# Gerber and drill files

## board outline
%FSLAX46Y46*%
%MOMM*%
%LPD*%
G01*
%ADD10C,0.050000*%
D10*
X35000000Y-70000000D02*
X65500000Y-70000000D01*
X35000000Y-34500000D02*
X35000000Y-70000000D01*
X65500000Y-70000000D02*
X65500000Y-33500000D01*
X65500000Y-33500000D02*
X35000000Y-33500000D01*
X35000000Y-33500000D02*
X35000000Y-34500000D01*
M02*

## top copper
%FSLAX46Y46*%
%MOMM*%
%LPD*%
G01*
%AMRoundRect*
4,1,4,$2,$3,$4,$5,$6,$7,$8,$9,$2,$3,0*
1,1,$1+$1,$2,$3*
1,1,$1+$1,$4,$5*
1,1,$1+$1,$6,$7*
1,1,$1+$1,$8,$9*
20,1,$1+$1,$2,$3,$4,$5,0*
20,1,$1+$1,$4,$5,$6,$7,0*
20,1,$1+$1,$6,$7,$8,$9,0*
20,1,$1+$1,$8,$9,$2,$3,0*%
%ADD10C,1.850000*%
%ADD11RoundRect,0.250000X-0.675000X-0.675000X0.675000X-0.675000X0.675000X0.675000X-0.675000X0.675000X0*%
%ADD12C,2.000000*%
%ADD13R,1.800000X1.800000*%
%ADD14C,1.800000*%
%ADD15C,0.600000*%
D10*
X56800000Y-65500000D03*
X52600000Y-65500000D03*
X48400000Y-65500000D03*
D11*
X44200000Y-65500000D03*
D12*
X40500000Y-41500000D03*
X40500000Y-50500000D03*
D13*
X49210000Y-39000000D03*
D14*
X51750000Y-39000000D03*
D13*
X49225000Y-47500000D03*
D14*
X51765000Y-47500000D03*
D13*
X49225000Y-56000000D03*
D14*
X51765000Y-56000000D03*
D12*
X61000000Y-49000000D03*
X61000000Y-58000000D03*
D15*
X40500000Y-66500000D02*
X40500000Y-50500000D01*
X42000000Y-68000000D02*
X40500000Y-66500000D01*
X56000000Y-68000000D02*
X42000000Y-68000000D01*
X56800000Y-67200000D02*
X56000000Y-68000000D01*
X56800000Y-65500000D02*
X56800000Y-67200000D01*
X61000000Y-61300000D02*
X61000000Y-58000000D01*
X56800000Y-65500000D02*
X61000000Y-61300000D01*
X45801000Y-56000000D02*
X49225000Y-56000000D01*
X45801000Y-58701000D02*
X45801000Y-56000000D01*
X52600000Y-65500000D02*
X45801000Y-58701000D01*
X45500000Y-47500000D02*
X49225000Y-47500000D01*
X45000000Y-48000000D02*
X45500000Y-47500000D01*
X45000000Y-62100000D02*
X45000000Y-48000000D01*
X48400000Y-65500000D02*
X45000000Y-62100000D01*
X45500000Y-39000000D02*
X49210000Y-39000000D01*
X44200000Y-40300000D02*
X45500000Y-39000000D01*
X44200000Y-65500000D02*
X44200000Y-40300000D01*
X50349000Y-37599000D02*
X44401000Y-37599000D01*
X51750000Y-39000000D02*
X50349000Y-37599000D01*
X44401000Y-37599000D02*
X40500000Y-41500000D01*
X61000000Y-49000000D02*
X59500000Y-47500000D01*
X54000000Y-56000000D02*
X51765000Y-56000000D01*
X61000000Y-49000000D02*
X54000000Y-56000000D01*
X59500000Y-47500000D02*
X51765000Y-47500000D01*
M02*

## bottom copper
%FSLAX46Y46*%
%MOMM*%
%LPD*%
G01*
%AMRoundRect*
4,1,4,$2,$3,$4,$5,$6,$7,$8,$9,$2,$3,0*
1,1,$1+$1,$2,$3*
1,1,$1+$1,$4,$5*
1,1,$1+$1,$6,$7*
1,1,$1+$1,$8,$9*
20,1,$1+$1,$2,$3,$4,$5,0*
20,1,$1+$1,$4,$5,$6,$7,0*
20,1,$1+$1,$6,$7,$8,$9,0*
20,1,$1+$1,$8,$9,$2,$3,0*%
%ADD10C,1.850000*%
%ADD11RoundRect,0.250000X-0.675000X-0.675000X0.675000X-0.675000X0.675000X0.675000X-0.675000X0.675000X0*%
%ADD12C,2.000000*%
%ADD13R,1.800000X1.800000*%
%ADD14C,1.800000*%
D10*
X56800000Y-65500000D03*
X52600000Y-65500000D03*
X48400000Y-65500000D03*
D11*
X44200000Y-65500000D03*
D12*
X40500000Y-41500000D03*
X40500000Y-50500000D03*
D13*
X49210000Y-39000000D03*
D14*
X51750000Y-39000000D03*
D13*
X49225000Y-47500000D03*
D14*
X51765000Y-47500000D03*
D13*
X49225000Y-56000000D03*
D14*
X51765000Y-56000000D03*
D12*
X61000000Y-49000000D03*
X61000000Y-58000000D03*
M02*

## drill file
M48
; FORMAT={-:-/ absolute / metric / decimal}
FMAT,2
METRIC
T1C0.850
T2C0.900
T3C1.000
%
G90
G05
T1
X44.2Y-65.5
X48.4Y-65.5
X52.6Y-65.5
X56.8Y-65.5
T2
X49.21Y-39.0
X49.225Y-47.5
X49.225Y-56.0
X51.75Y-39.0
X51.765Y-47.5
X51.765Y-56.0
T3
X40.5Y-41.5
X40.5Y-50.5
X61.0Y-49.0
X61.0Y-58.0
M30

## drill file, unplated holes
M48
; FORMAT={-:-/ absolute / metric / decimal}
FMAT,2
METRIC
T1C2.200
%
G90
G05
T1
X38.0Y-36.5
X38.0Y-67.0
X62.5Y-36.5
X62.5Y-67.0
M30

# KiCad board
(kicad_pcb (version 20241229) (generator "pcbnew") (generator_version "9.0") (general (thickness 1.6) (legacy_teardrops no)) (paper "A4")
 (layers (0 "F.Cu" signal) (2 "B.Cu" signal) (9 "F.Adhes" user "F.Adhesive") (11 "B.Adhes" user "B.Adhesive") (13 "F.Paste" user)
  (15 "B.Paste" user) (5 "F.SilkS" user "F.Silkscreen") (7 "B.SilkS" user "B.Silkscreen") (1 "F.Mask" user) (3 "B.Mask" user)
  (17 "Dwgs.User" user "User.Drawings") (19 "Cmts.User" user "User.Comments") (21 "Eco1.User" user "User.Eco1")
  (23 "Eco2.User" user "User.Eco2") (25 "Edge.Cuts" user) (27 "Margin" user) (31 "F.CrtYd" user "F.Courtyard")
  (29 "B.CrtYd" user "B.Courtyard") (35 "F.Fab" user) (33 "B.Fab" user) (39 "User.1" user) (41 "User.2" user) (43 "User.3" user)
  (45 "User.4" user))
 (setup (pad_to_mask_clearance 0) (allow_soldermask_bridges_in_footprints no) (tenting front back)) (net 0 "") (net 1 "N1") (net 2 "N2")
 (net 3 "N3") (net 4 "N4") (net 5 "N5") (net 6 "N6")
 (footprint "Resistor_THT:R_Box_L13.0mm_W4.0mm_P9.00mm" (layer "F.Cu") (at 40.5 41.5 -90)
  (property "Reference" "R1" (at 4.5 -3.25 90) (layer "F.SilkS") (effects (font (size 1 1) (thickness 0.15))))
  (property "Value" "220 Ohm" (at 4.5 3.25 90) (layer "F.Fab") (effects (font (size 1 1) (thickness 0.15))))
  (pad "1" thru_hole circle (at 0 0 270) (size 2 2) (drill 1) (layers "*.Cu" "*.Mask") (remove_unused_layers no) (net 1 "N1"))
  (pad "2" thru_hole circle (at 9 0 270) (size 2 2) (drill 1) (layers "*.Cu" "*.Mask") (remove_unused_layers no) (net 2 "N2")))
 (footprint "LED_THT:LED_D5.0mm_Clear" (layer "F.Cu") (at 49.21 39)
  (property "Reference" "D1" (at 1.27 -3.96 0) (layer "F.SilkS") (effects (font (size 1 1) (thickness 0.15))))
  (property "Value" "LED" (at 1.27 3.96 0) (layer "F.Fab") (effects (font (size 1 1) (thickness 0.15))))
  (pad "1" thru_hole rect (at 0 0) (size 1.8 1.8) (drill 0.9) (layers "*.Cu" "*.Mask") (remove_unused_layers no) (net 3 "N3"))
  (pad "2" thru_hole circle (at 2.54 0) (size 1.8 1.8) (drill 0.9) (layers "*.Cu" "*.Mask") (remove_unused_layers no) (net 1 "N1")))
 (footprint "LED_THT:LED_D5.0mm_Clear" (layer "F.Cu") (at 49.225 47.5)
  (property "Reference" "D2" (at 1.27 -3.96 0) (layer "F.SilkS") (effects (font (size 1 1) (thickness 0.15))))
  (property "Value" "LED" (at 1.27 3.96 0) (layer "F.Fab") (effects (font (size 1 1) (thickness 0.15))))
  (pad "1" thru_hole rect (at 0 0) (size 1.8 1.8) (drill 0.9) (layers "*.Cu" "*.Mask") (remove_unused_layers no) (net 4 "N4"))
  (pad "2" thru_hole circle (at 2.54 0) (size 1.8 1.8) (drill 0.9) (layers "*.Cu" "*.Mask") (remove_unused_layers no) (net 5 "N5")))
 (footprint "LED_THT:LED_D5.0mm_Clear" (layer "F.Cu") (at 49.225 56)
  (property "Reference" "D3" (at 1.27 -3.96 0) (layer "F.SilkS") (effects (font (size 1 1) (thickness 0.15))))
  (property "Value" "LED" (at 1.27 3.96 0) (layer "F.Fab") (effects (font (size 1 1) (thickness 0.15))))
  (pad "1" thru_hole rect (at 0 0) (size 1.8 1.8) (drill 0.9) (layers "*.Cu" "*.Mask") (remove_unused_layers no) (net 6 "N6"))
  (pad "2" thru_hole circle (at 2.54 0) (size 1.8 1.8) (drill 0.9) (layers "*.Cu" "*.Mask") (remove_unused_layers no) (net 5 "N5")))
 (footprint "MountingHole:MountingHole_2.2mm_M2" (layer "F.Cu") (at 38 36.5)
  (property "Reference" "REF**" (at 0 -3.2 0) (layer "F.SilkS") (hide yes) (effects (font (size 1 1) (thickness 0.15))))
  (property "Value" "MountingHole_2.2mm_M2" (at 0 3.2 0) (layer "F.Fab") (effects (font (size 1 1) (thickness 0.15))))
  (pad "" np_thru_hole circle (at 0 0) (size 2.2 2.2) (drill 2.2) (layers "*.Cu" "*.Mask")))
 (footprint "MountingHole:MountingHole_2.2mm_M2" (layer "F.Cu") (at 38 67)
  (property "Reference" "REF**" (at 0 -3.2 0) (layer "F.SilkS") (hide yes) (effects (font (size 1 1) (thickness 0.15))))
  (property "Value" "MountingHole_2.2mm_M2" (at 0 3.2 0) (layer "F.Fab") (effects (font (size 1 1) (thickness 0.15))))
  (pad "" np_thru_hole circle (at 0 0) (size 2.2 2.2) (drill 2.2) (layers "*.Cu" "*.Mask")))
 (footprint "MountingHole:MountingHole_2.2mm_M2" (layer "F.Cu") (at 62.5 36.5)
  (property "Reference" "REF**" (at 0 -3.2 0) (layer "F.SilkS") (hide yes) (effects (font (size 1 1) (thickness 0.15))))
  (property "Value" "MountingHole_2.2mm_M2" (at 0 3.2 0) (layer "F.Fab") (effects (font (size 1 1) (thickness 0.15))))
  (pad "" np_thru_hole circle (at 0 0) (size 2.2 2.2) (drill 2.2) (layers "*.Cu" "*.Mask")))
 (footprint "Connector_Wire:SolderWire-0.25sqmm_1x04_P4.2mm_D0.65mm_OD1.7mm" (layer "F.Cu") (at 44.2 65.5)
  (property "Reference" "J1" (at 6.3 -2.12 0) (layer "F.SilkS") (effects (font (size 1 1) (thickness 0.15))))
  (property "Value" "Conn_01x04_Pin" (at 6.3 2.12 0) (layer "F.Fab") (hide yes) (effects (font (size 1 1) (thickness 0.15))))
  (pad "1" thru_hole roundrect (at 0 0) (size 1.85 1.85) (drill 0.85) (layers "*.Cu" "*.Mask") (remove_unused_layers no)
   (roundrect_rratio 0.135135) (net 3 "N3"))
  (pad "2" thru_hole circle (at 4.2 0) (size 1.85 1.85) (drill 0.85) (layers "*.Cu" "*.Mask") (remove_unused_layers no) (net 4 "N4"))
  (pad "3" thru_hole circle (at 8.4 0) (size 1.85 1.85) (drill 0.85) (layers "*.Cu" "*.Mask") (remove_unused_layers no) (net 6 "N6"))
  (pad "4" thru_hole circle (at 12.6 0) (size 1.85 1.85) (drill 0.85) (layers "*.Cu" "*.Mask") (remove_unused_layers no) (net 2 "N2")))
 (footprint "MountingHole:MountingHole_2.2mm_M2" (layer "F.Cu") (at 62.5 67)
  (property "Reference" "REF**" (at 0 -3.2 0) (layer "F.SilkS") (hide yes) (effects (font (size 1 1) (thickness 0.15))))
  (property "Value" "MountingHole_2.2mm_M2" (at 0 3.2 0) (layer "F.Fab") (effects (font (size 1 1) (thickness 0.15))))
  (pad "" np_thru_hole circle (at 0 0) (size 2.2 2.2) (drill 2.2) (layers "*.Cu" "*.Mask")))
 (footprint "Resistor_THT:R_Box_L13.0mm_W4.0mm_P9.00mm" (layer "F.Cu") (at 61 49 -90)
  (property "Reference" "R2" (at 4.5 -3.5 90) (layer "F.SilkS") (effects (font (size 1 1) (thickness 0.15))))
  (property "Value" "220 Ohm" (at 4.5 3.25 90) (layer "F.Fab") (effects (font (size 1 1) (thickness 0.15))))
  (pad "1" thru_hole circle (at 0 0 270) (size 2 2) (drill 1) (layers "*.Cu" "*.Mask") (remove_unused_layers no) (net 5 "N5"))
  (pad "2" thru_hole circle (at 9 0 270) (size 2 2) (drill 1) (layers "*.Cu" "*.Mask") (remove_unused_layers no) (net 2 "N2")))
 (gr_line (start 35 70) (end 65.5 70) (stroke (width 0.05) (type default)) (layer "Edge.Cuts"))
 (gr_line (start 35 34.5) (end 35 70) (stroke (width 0.05) (type default)) (layer "Edge.Cuts"))
 (gr_line (start 65.5 70) (end 65.5 33.5) (stroke (width 0.05) (type default)) (layer "Edge.Cuts"))
 (gr_line (start 65.5 33.5) (end 35 33.5) (stroke (width 0.05) (type default)) (layer "Edge.Cuts"))
 (gr_line (start 35 33.5) (end 35 34.5) (stroke (width 0.05) (type default)) (layer "Edge.Cuts"))
 (segment (start 44.2 40.3) (end 45.5 39) (width 0.6) (layer "F.Cu") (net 3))
 (segment (start 44.2 65.5) (end 44.2 40.3) (width 0.6) (layer "F.Cu") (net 3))
 (segment (start 45.5 39) (end 49.21 39) (width 0.6) (layer "F.Cu") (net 3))
 (segment (start 50.349 37.599) (end 44.401 37.599) (width 0.6) (layer "F.Cu") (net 1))
 (segment (start 51.75 39) (end 50.349 37.599) (width 0.6) (layer "F.Cu") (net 1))
 (segment (start 44.401 37.599) (end 40.5 41.5) (width 0.6) (layer "F.Cu") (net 1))
 (segment (start 48.4 65.5) (end 45 62.1) (width 0.6) (layer "F.Cu") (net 4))
 (segment (start 45 62.1) (end 45 48) (width 0.6) (layer "F.Cu") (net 4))
 (segment (start 45.5 47.5) (end 49.225 47.5) (width 0.6) (layer "F.Cu") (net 4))
 (segment (start 45 48) (end 45.5 47.5) (width 0.6) (layer "F.Cu") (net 4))
 (segment (start 61 49) (end 59.5 47.5) (width 0.6) (layer "F.Cu") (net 5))
 (segment (start 54 56) (end 51.765 56) (width 0.6) (layer "F.Cu") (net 5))
 (segment (start 61 49) (end 54 56) (width 0.6) (layer "F.Cu") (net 5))
 (segment (start 59.5 47.5) (end 51.765 47.5) (width 0.6) (layer "F.Cu") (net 5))
 (segment (start 45.801 56) (end 49.225 56) (width 0.6) (layer "F.Cu") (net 6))
 (segment (start 45.801 58.701) (end 45.801 56) (width 0.6) (layer "F.Cu") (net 6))
 (segment (start 52.6 65.5) (end 45.801 58.701) (width 0.6) (layer "F.Cu") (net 6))
 (segment (start 42 68) (end 40.5 66.5) (width 0.6) (layer "F.Cu") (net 2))
 (segment (start 56.8 67.2) (end 56 68) (width 0.6) (layer "F.Cu") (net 2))
 (segment (start 61 61.3) (end 61 58) (width 0.6) (layer "F.Cu") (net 2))
 (segment (start 56 68) (end 42 68) (width 0.6) (layer "F.Cu") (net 2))
 (segment (start 40.5 66.5) (end 40.5 50.5) (width 0.6) (layer "F.Cu") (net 2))
 (segment (start 56.8 65.5) (end 56.8 67.2) (width 0.6) (layer "F.Cu") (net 2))
 (segment (start 56.8 65.5) (end 61 61.3) (width 0.6) (layer "F.Cu") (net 2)))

